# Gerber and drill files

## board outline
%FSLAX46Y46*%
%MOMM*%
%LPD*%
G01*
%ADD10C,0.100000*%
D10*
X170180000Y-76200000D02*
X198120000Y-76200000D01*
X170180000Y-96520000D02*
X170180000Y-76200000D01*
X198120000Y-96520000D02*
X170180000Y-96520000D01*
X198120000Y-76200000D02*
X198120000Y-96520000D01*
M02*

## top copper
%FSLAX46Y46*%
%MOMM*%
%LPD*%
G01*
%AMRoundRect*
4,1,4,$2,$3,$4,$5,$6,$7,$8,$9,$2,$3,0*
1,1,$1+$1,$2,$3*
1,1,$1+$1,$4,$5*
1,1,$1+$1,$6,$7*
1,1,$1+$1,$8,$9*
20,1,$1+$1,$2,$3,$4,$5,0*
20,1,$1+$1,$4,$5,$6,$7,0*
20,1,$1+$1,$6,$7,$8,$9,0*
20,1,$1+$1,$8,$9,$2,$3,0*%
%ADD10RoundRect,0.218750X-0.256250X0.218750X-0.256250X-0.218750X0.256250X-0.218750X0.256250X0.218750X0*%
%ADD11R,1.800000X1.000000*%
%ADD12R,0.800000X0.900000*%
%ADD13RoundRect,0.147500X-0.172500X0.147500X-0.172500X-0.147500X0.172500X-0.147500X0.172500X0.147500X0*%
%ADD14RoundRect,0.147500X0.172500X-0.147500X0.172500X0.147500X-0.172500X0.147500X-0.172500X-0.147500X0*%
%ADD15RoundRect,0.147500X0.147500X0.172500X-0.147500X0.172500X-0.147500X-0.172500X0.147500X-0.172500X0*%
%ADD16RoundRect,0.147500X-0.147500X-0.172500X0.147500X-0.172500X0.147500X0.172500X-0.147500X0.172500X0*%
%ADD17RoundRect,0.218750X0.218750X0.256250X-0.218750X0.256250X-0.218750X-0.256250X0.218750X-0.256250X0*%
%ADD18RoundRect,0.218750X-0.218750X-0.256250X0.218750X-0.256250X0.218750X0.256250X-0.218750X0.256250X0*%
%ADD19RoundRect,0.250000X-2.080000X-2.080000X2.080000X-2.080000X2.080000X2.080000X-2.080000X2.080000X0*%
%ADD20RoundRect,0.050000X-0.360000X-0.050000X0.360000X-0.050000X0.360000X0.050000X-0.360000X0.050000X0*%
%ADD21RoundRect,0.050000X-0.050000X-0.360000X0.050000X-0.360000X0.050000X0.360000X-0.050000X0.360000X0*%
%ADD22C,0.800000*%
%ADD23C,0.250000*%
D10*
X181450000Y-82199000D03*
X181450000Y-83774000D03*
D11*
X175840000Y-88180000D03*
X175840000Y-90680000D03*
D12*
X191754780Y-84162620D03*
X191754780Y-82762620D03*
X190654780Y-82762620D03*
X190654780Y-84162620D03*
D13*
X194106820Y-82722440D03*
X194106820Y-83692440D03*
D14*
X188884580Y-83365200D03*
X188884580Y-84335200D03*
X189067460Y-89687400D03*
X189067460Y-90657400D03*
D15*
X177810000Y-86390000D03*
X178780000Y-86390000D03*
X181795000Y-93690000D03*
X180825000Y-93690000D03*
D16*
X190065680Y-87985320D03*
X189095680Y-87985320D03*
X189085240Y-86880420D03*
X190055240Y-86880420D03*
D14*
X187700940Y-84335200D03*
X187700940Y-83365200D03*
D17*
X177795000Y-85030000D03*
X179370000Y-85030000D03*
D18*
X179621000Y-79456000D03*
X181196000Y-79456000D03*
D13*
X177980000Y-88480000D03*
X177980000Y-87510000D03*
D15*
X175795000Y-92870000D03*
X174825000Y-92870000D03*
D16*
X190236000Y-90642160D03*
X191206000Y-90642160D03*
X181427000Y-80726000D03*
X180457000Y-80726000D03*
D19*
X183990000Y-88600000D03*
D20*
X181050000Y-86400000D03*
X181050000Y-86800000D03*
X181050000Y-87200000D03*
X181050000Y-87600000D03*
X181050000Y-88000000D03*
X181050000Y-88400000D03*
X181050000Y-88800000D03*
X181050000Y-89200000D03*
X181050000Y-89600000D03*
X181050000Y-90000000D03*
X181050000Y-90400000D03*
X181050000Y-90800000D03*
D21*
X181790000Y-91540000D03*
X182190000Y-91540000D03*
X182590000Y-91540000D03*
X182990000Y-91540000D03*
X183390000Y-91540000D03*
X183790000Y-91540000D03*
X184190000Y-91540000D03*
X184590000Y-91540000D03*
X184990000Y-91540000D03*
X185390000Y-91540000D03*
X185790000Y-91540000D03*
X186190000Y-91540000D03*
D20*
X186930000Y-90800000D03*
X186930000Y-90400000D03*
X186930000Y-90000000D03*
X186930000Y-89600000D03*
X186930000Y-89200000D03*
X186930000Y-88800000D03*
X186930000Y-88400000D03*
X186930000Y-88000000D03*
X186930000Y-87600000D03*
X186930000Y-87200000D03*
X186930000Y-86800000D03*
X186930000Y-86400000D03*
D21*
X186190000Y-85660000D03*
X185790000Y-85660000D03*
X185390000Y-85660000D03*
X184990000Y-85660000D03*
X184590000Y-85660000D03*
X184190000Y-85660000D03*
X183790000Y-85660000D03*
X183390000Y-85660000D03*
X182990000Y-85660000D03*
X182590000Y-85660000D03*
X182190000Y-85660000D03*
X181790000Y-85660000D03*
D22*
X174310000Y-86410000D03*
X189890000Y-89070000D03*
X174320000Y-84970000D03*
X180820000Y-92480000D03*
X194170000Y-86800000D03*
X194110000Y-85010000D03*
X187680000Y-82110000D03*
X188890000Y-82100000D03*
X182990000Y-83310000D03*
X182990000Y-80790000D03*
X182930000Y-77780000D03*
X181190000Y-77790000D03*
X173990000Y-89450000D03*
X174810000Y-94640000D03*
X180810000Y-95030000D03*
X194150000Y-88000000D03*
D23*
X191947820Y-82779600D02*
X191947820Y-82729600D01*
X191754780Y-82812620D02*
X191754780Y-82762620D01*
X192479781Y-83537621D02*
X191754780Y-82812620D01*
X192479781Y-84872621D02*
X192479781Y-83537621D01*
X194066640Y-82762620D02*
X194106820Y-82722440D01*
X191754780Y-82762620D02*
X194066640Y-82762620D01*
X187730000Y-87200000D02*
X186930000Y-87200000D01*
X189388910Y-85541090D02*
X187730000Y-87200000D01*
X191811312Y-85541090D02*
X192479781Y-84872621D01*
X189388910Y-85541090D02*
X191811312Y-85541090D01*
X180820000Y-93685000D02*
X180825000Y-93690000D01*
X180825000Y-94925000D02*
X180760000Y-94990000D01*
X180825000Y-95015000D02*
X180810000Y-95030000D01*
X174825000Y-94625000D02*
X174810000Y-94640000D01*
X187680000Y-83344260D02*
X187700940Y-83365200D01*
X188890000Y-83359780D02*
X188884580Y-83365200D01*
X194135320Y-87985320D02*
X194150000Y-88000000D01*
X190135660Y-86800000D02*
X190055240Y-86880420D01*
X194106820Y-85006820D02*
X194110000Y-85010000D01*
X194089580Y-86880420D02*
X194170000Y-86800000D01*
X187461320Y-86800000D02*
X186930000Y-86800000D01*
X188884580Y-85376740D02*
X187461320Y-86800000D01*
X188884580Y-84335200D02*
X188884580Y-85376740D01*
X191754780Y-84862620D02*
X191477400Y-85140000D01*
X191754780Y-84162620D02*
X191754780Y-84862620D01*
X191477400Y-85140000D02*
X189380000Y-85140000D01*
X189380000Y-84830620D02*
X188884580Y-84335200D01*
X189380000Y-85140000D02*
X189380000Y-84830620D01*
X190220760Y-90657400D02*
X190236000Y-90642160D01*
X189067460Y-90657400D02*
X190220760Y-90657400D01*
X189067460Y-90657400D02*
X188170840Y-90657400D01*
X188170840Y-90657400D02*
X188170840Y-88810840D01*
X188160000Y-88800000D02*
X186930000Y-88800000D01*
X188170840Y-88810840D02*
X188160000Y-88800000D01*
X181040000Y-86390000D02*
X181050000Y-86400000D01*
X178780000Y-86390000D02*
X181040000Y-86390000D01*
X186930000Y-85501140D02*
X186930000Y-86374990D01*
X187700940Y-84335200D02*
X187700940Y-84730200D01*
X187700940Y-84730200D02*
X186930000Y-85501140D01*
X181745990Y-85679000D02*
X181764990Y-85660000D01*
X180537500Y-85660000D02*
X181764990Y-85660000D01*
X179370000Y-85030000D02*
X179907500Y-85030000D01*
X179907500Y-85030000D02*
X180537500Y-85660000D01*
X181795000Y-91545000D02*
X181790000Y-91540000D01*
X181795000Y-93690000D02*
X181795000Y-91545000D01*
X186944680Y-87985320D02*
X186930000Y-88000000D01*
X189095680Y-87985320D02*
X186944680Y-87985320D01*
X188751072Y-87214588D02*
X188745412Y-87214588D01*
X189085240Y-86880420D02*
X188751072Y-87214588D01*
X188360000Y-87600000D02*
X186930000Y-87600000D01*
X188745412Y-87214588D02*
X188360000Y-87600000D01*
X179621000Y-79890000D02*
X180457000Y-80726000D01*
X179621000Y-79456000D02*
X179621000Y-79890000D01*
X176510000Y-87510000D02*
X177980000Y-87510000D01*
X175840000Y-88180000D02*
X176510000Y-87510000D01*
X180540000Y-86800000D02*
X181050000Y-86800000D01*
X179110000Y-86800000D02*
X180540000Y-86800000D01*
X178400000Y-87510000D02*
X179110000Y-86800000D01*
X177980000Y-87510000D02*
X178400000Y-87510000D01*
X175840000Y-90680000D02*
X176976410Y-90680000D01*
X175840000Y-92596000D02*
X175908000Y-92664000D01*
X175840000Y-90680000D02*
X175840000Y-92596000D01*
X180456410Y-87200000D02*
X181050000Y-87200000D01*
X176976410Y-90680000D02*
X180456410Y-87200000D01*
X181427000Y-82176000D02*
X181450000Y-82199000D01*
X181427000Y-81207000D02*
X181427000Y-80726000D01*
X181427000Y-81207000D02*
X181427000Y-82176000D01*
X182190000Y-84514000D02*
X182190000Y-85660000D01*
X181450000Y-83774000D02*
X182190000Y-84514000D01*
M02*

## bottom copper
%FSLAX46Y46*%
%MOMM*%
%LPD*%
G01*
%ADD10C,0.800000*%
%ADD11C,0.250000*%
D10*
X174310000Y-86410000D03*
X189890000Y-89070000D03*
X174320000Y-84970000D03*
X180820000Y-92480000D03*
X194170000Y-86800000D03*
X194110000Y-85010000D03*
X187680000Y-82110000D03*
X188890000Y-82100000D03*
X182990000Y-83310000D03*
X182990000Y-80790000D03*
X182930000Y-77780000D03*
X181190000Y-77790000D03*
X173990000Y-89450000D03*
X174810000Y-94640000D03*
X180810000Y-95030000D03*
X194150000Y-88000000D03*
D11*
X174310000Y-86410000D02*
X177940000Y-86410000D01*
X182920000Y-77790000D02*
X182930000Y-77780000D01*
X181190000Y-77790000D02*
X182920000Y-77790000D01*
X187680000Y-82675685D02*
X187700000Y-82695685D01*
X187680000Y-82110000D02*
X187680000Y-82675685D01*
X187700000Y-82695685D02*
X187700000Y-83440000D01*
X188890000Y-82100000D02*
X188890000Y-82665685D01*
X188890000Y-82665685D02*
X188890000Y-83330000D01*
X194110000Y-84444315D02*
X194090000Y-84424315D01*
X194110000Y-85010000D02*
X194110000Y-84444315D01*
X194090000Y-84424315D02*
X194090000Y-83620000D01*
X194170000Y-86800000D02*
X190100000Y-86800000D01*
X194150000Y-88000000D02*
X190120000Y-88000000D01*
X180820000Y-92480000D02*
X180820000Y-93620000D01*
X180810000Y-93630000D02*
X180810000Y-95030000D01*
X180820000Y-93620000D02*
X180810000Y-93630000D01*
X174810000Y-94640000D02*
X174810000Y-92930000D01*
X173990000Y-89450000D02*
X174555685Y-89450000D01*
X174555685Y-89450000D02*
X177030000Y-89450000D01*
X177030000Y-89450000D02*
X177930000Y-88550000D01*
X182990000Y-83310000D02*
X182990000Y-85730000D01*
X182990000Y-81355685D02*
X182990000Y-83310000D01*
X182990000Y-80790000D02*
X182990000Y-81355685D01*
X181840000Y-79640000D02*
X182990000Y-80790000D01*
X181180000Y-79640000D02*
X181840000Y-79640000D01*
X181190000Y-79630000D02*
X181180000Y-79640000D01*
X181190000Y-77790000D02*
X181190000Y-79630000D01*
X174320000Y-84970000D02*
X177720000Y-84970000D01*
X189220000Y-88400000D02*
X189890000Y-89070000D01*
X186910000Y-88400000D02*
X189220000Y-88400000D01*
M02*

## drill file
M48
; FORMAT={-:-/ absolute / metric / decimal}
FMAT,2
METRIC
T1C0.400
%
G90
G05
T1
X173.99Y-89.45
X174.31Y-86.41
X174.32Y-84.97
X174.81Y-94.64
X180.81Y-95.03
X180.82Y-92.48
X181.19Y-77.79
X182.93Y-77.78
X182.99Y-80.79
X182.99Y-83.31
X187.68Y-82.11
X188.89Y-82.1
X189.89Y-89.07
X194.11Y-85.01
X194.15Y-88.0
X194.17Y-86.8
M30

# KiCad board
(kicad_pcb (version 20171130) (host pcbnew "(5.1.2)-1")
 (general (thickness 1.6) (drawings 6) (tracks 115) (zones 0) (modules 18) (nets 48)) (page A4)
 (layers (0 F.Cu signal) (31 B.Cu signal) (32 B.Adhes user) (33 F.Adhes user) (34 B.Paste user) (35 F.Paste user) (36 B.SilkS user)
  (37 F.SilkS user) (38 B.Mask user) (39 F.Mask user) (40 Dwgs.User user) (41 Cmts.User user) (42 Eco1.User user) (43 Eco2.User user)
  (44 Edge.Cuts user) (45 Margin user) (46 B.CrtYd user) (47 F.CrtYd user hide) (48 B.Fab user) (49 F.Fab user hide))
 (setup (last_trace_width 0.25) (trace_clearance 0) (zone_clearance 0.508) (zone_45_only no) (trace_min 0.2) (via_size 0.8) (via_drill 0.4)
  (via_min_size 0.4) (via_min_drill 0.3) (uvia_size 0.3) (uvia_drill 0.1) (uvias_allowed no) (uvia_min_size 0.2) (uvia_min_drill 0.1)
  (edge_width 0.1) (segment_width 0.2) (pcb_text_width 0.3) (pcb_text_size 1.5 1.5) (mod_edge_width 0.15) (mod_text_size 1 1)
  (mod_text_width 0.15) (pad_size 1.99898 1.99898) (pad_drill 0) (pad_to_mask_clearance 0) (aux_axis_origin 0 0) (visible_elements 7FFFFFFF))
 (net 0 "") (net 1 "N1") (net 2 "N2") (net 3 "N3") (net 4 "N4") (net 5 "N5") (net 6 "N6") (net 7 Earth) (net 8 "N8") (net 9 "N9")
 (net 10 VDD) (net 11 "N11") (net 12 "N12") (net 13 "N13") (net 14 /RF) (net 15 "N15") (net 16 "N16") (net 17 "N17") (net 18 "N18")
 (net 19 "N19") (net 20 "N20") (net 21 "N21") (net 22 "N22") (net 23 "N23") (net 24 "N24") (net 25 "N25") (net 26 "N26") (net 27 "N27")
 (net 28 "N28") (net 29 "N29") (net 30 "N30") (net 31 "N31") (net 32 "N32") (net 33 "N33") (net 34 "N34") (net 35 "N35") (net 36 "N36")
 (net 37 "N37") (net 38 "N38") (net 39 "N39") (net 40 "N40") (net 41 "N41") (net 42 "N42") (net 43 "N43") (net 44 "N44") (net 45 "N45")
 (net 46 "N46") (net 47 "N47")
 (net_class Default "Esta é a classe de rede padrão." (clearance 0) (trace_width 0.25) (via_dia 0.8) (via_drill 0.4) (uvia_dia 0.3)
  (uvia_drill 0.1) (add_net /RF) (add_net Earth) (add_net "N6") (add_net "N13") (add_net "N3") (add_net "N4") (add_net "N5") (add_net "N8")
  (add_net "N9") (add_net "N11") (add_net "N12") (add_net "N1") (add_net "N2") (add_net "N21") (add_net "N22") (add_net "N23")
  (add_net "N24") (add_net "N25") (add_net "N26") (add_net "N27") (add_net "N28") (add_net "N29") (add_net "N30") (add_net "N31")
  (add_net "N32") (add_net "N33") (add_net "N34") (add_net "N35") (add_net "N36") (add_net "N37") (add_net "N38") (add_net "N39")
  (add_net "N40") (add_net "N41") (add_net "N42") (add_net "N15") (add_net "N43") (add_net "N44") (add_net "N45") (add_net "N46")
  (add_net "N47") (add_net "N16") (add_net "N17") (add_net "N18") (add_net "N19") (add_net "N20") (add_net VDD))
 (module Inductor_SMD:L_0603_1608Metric (layer F.Cu) (at 181.45 82.9865 270)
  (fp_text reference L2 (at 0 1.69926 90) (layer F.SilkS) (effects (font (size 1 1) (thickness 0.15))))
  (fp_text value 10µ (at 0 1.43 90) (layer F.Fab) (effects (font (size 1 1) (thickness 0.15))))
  (pad 1 smd roundrect (at -0.7875 0 270) (size 0.875 0.95) (layers F.Cu F.Paste F.Mask) (roundrect_rratio 0.25) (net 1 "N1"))
  (pad 2 smd roundrect (at 0.7875 0 270) (size 0.875 0.95) (layers F.Cu F.Paste F.Mask) (roundrect_rratio 0.25) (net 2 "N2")))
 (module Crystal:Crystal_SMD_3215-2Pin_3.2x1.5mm (layer F.Cu) (at 175.84 89.43 90)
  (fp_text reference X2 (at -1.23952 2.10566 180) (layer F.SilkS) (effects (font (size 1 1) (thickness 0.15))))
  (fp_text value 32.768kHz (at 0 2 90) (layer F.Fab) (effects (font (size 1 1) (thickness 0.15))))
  (pad 1 smd rect (at 1.25 0 90) (size 1 1.8) (layers F.Cu F.Paste F.Mask) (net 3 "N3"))
  (pad 2 smd rect (at -1.25 0 90) (size 1 1.8) (layers F.Cu F.Paste F.Mask) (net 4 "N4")))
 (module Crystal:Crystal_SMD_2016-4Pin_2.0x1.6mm (layer F.Cu) (at 191.20478 83.46262 90)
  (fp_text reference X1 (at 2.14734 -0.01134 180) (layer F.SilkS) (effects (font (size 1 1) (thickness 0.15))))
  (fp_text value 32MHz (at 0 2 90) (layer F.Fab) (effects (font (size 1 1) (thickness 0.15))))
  (pad 1 smd rect (at -0.7 0.55 90) (size 0.9 0.8) (layers F.Cu F.Paste F.Mask) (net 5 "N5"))
  (pad 2 smd rect (at 0.7 0.55 90) (size 0.9 0.8) (layers F.Cu F.Paste F.Mask) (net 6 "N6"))
  (pad 3 smd rect (at 0.7 -0.55 90) (size 0.9 0.8) (layers F.Cu F.Paste F.Mask))
  (pad 4 smd rect (at -0.7 -0.55 90) (size 0.9 0.8) (layers F.Cu F.Paste F.Mask)))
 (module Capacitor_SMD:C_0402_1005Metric (layer F.Cu) (at 194.10682 83.20744 270)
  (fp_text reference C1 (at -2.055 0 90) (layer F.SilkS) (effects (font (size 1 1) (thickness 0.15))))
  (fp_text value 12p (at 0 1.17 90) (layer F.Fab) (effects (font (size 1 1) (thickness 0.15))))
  (pad 1 smd roundrect (at -0.485 0 270) (size 0.59 0.64) (layers F.Cu F.Paste F.Mask) (roundrect_rratio 0.25) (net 6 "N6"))
  (pad 2 smd roundrect (at 0.485 0 270) (size 0.59 0.64) (layers F.Cu F.Paste F.Mask) (roundrect_rratio 0.25) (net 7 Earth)))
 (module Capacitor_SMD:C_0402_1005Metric (layer F.Cu) (at 188.88458 83.8502 90)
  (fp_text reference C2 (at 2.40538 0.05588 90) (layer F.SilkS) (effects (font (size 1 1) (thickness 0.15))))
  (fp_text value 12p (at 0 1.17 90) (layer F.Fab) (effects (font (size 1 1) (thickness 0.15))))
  (pad 2 smd roundrect (at 0.485 0 90) (size 0.59 0.64) (layers F.Cu F.Paste F.Mask) (roundrect_rratio 0.25) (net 7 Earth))
  (pad 1 smd roundrect (at -0.485 0 90) (size 0.59 0.64) (layers F.Cu F.Paste F.Mask) (roundrect_rratio 0.25) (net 5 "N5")))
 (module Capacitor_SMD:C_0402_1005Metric (layer F.Cu) (at 189.06746 90.1724 90)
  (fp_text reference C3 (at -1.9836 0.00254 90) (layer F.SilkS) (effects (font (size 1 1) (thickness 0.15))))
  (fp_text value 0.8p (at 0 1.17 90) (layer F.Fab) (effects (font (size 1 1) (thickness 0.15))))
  (pad 2 smd roundrect (at 0.485 0 90) (size 0.59 0.64) (layers F.Cu F.Paste F.Mask) (roundrect_rratio 0.25) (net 7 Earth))
  (pad 1 smd roundrect (at -0.485 0 90) (size 0.59 0.64) (layers F.Cu F.Paste F.Mask) (roundrect_rratio 0.25) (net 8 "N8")))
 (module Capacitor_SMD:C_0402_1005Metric (layer F.Cu) (at 178.295 86.39 180)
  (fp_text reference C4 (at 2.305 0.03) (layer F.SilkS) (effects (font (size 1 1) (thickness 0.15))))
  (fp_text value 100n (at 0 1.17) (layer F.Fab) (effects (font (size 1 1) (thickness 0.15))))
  (pad 2 smd roundrect (at 0.485 0 180) (size 0.59 0.64) (layers F.Cu F.Paste F.Mask) (roundrect_rratio 0.25) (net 7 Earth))
  (pad 1 smd roundrect (at -0.485 0 180) (size 0.59 0.64) (layers F.Cu F.Paste F.Mask) (roundrect_rratio 0.25) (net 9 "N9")))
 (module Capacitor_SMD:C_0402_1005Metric (layer F.Cu) (at 181.31 93.69 180)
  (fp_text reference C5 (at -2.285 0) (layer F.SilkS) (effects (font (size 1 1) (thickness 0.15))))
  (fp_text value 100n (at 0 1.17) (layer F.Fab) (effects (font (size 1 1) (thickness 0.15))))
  (pad 1 smd roundrect (at -0.485 0 180) (size 0.59 0.64) (layers F.Cu F.Paste F.Mask) (roundrect_rratio 0.25) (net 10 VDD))
  (pad 2 smd roundrect (at 0.485 0 180) (size 0.59 0.64) (layers F.Cu F.Paste F.Mask) (roundrect_rratio 0.25) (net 7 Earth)))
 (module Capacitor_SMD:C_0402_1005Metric (layer F.Cu) (at 189.58068 87.98532)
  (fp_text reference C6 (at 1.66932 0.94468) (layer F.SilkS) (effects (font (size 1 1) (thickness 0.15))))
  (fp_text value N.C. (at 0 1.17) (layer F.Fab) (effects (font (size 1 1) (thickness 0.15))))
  (pad 2 smd roundrect (at 0.485 0) (size 0.59 0.64) (layers F.Cu F.Paste F.Mask) (roundrect_rratio 0.25) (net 7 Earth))
  (pad 1 smd roundrect (at -0.485 0) (size 0.59 0.64) (layers F.Cu F.Paste F.Mask) (roundrect_rratio 0.25) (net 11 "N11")))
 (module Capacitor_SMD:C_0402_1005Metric (layer F.Cu) (at 189.57024 86.88042)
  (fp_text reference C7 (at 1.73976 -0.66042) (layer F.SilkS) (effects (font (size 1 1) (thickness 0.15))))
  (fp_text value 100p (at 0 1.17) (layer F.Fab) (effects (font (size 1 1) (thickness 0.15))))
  (pad 1 smd roundrect (at -0.485 0) (size 0.59 0.64) (layers F.Cu F.Paste F.Mask) (roundrect_rratio 0.25) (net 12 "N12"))
  (pad 2 smd roundrect (at 0.485 0) (size 0.59 0.64) (layers F.Cu F.Paste F.Mask) (roundrect_rratio 0.25) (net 7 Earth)))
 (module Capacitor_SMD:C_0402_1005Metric (layer F.Cu) (at 187.70094 83.8502 90)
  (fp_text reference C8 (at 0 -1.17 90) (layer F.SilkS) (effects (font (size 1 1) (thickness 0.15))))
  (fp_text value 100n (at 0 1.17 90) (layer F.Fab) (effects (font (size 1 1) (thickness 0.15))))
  (pad 1 smd roundrect (at -0.485 0 90) (size 0.59 0.64) (layers F.Cu F.Paste F.Mask) (roundrect_rratio 0.25) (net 10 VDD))
  (pad 2 smd roundrect (at 0.485 0 90) (size 0.59 0.64) (layers F.Cu F.Paste F.Mask) (roundrect_rratio 0.25) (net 7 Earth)))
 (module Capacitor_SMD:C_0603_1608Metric (layer F.Cu) (at 178.5825 85.03 180)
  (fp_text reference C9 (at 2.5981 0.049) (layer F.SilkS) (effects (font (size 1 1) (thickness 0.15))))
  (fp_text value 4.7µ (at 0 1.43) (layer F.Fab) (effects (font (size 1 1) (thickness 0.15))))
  (pad 2 smd roundrect (at 0.7875 0 180) (size 0.875 0.95) (layers F.Cu F.Paste F.Mask) (roundrect_rratio 0.25) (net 7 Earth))
  (pad 1 smd roundrect (at -0.7875 0 180) (size 0.875 0.95) (layers F.Cu F.Paste F.Mask) (roundrect_rratio 0.25) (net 10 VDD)))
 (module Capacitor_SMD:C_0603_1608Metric (layer F.Cu) (at 180.4085 79.456)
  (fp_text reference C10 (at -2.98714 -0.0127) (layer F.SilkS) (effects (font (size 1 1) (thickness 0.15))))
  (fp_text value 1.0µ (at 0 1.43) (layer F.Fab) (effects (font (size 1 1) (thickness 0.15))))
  (pad 1 smd roundrect (at -0.7875 0) (size 0.875 0.95) (layers F.Cu F.Paste F.Mask) (roundrect_rratio 0.25) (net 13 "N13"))
  (pad 2 smd roundrect (at 0.7875 0) (size 0.875 0.95) (layers F.Cu F.Paste F.Mask) (roundrect_rratio 0.25) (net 7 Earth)))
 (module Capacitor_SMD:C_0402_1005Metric (layer F.Cu) (at 177.98 87.995 270)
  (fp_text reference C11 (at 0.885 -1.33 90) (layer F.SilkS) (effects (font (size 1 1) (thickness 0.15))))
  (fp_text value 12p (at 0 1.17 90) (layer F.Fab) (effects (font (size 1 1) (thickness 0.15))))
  (pad 2 smd roundrect (at 0.485 0 270) (size 0.59 0.64) (layers F.Cu F.Paste F.Mask) (roundrect_rratio 0.25) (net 7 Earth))
  (pad 1 smd roundrect (at -0.485 0 270) (size 0.59 0.64) (layers F.Cu F.Paste F.Mask) (roundrect_rratio 0.25) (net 3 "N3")))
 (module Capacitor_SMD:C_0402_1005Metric (layer F.Cu) (at 175.31 92.87 180)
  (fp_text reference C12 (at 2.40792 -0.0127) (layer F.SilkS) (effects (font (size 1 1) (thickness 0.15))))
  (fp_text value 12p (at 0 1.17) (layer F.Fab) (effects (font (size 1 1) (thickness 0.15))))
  (pad 1 smd roundrect (at -0.485 0 180) (size 0.59 0.64) (layers F.Cu F.Paste F.Mask) (roundrect_rratio 0.25) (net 4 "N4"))
  (pad 2 smd roundrect (at 0.485 0 180) (size 0.59 0.64) (layers F.Cu F.Paste F.Mask) (roundrect_rratio 0.25) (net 7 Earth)))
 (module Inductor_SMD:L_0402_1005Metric (layer F.Cu) (at 190.721 90.64216)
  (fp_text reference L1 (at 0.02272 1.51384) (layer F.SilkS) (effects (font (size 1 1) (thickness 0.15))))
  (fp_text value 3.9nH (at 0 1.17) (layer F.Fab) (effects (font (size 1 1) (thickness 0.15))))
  (pad 1 smd roundrect (at -0.485 0) (size 0.59 0.64) (layers F.Cu F.Paste F.Mask) (roundrect_rratio 0.25) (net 8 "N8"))
  (pad 2 smd roundrect (at 0.485 0) (size 0.59 0.64) (layers F.Cu F.Paste F.Mask) (roundrect_rratio 0.25) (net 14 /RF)))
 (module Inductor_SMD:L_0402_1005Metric (layer F.Cu) (at 180.942 80.726)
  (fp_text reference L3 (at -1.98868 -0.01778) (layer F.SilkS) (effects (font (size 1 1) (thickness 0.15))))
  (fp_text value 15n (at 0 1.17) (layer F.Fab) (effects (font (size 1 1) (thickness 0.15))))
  (pad 2 smd roundrect (at 0.485 0) (size 0.59 0.64) (layers F.Cu F.Paste F.Mask) (roundrect_rratio 0.25) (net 1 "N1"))
  (pad 1 smd roundrect (at -0.485 0) (size 0.59 0.64) (layers F.Cu F.Paste F.Mask) (roundrect_rratio 0.25) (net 13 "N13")))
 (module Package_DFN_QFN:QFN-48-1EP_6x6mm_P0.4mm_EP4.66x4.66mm (layer F.Cu) (at 183.99 88.6)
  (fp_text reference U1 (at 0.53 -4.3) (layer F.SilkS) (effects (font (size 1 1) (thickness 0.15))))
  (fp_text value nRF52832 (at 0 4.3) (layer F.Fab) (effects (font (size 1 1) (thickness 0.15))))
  (pad 49 smd roundrect (at 0 0) (size 4.66 4.66) (layers F.Cu F.Mask) (roundrect_rratio 0.053648))
  (pad "" smd roundrect (at -1.55 -1.55) (size 1.25 1.25) (layers F.Paste) (roundrect_rratio 0.2))
  (pad "" smd roundrect (at -1.55 0) (size 1.25 1.25) (layers F.Paste) (roundrect_rratio 0.2))
  (pad "" smd roundrect (at -1.55 1.55) (size 1.25 1.25) (layers F.Paste) (roundrect_rratio 0.2))
  (pad "" smd roundrect (at 0 -1.55) (size 1.25 1.25) (layers F.Paste) (roundrect_rratio 0.2))
  (pad "" smd roundrect (at 0 0) (size 1.25 1.25) (layers F.Paste) (roundrect_rratio 0.2))
  (pad "" smd roundrect (at 0 1.55) (size 1.25 1.25) (layers F.Paste) (roundrect_rratio 0.2))
  (pad "" smd roundrect (at 1.55 -1.55) (size 1.25 1.25) (layers F.Paste) (roundrect_rratio 0.2))
  (pad "" smd roundrect (at 1.55 0) (size 1.25 1.25) (layers F.Paste) (roundrect_rratio 0.2))
  (pad "" smd roundrect (at 1.55 1.55) (size 1.25 1.25) (layers F.Paste) (roundrect_rratio 0.2))
  (pad 1 smd roundrect (at -2.94 -2.2) (size 0.82 0.2) (layers F.Cu F.Paste F.Mask) (roundrect_rratio 0.25) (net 9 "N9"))
  (pad 2 smd roundrect (at -2.94 -1.8) (size 0.82 0.2) (layers F.Cu F.Paste F.Mask) (roundrect_rratio 0.25) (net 3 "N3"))
  (pad 3 smd roundrect (at -2.94 -1.4) (size 0.82 0.2) (layers F.Cu F.Paste F.Mask) (roundrect_rratio 0.25) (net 4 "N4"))
  (pad 4 smd roundrect (at -2.94 -1) (size 0.82 0.2) (layers F.Cu F.Paste F.Mask) (roundrect_rratio 0.25) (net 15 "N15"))
  (pad 5 smd roundrect (at -2.94 -0.6) (size 0.82 0.2) (layers F.Cu F.Paste F.Mask) (roundrect_rratio 0.25) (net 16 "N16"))
  (pad 6 smd roundrect (at -2.94 -0.2) (size 0.82 0.2) (layers F.Cu F.Paste F.Mask) (roundrect_rratio 0.25) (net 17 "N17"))
  (pad 7 smd roundrect (at -2.94 0.2) (size 0.82 0.2) (layers F.Cu F.Paste F.Mask) (roundrect_rratio 0.25) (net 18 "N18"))
  (pad 8 smd roundrect (at -2.94 0.6) (size 0.82 0.2) (layers F.Cu F.Paste F.Mask) (roundrect_rratio 0.25) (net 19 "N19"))
  (pad 9 smd roundrect (at -2.94 1) (size 0.82 0.2) (layers F.Cu F.Paste F.Mask) (roundrect_rratio 0.25) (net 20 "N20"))
  (pad 10 smd roundrect (at -2.94 1.4) (size 0.82 0.2) (layers F.Cu F.Paste F.Mask) (roundrect_rratio 0.25) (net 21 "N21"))
  (pad 11 smd roundrect (at -2.94 1.8) (size 0.82 0.2) (layers F.Cu F.Paste F.Mask) (roundrect_rratio 0.25) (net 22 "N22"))
  (pad 12 smd roundrect (at -2.94 2.2) (size 0.82 0.2) (layers F.Cu F.Paste F.Mask) (roundrect_rratio 0.25) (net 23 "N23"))
  (pad 13 smd roundrect (at -2.2 2.94) (size 0.2 0.82) (layers F.Cu F.Paste F.Mask) (roundrect_rratio 0.25) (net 10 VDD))
  (pad 14 smd roundrect (at -1.8 2.94) (size 0.2 0.82) (layers F.Cu F.Paste F.Mask) (roundrect_rratio 0.25) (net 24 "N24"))
  (pad 15 smd roundrect (at -1.4 2.94) (size 0.2 0.82) (layers F.Cu F.Paste F.Mask) (roundrect_rratio 0.25) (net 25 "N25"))
  (pad 16 smd roundrect (at -1 2.94) (size 0.2 0.82) (layers F.Cu F.Paste F.Mask) (roundrect_rratio 0.25) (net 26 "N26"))
  (pad 17 smd roundrect (at -0.6 2.94) (size 0.2 0.82) (layers F.Cu F.Paste F.Mask) (roundrect_rratio 0.25) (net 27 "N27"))
  (pad 18 smd roundrect (at -0.2 2.94) (size 0.2 0.82) (layers F.Cu F.Paste F.Mask) (roundrect_rratio 0.25) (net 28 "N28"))
  (pad 19 smd roundrect (at 0.2 2.94) (size 0.2 0.82) (layers F.Cu F.Paste F.Mask) (roundrect_rratio 0.25) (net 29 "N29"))
  (pad 20 smd roundrect (at 0.6 2.94) (size 0.2 0.82) (layers F.Cu F.Paste F.Mask) (roundrect_rratio 0.25) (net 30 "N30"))
  (pad 21 smd roundrect (at 1 2.94) (size 0.2 0.82) (layers F.Cu F.Paste F.Mask) (roundrect_rratio 0.25) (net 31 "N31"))
  (pad 22 smd roundrect (at 1.4 2.94) (size 0.2 0.82) (layers F.Cu F.Paste F.Mask) (roundrect_rratio 0.25) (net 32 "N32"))
  (pad 23 smd roundrect (at 1.8 2.94) (size 0.2 0.82) (layers F.Cu F.Paste F.Mask) (roundrect_rratio 0.25) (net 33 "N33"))
  (pad 24 smd roundrect (at 2.2 2.94) (size 0.2 0.82) (layers F.Cu F.Paste F.Mask) (roundrect_rratio 0.25) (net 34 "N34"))
  (pad 25 smd roundrect (at 2.94 2.2) (size 0.82 0.2) (layers F.Cu F.Paste F.Mask) (roundrect_rratio 0.25) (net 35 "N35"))
  (pad 26 smd roundrect (at 2.94 1.8) (size 0.82 0.2) (layers F.Cu F.Paste F.Mask) (roundrect_rratio 0.25) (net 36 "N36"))
  (pad 27 smd roundrect (at 2.94 1.4) (size 0.82 0.2) (layers F.Cu F.Paste F.Mask) (roundrect_rratio 0.25) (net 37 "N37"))
  (pad 28 smd roundrect (at 2.94 1) (size 0.82 0.2) (layers F.Cu F.Paste F.Mask) (roundrect_rratio 0.25) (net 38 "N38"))
  (pad 29 smd roundrect (at 2.94 0.6) (size 0.82 0.2) (layers F.Cu F.Paste F.Mask) (roundrect_rratio 0.25) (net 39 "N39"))
  (pad 30 smd roundrect (at 2.94 0.2) (size 0.82 0.2) (layers F.Cu F.Paste F.Mask) (roundrect_rratio 0.25) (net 8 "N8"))
  (pad 31 smd roundrect (at 2.94 -0.2) (size 0.82 0.2) (layers F.Cu F.Paste F.Mask) (roundrect_rratio 0.25) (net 7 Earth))
  (pad 32 smd roundrect (at 2.94 -0.6) (size 0.82 0.2) (layers F.Cu F.Paste F.Mask) (roundrect_rratio 0.25) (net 11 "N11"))
  (pad 33 smd roundrect (at 2.94 -1) (size 0.82 0.2) (layers F.Cu F.Paste F.Mask) (roundrect_rratio 0.25) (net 12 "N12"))
  (pad 34 smd roundrect (at 2.94 -1.4) (size 0.82 0.2) (layers F.Cu F.Paste F.Mask) (roundrect_rratio 0.25) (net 6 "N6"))
  (pad 35 smd roundrect (at 2.94 -1.8) (size 0.82 0.2) (layers F.Cu F.Paste F.Mask) (roundrect_rratio 0.25) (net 5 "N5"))
  (pad 36 smd roundrect (at 2.94 -2.2) (size 0.82 0.2) (layers F.Cu F.Paste F.Mask) (roundrect_rratio 0.25) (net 10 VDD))
  (pad 37 smd roundrect (at 2.2 -2.94) (size 0.2 0.82) (layers F.Cu F.Paste F.Mask) (roundrect_rratio 0.25) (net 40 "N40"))
  (pad 38 smd roundrect (at 1.8 -2.94) (size 0.2 0.82) (layers F.Cu F.Paste F.Mask) (roundrect_rratio 0.25) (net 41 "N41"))
  (pad 39 smd roundrect (at 1.4 -2.94) (size 0.2 0.82) (layers F.Cu F.Paste F.Mask) (roundrect_rratio 0.25) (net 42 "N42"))
  (pad 40 smd roundrect (at 1 -2.94) (size 0.2 0.82) (layers F.Cu F.Paste F.Mask) (roundrect_rratio 0.25) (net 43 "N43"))
  (pad 41 smd roundrect (at 0.6 -2.94) (size 0.2 0.82) (layers F.Cu F.Paste F.Mask) (roundrect_rratio 0.25) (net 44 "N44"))
  (pad 42 smd roundrect (at 0.2 -2.94) (size 0.2 0.82) (layers F.Cu F.Paste F.Mask) (roundrect_rratio 0.25) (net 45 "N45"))
  (pad 43 smd roundrect (at -0.2 -2.94) (size 0.2 0.82) (layers F.Cu F.Paste F.Mask) (roundrect_rratio 0.25) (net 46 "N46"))
  (pad 44 smd roundrect (at -0.6 -2.94) (size 0.2 0.82) (layers F.Cu F.Paste F.Mask) (roundrect_rratio 0.25) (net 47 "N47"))
  (pad 45 smd roundrect (at -1 -2.94) (size 0.2 0.82) (layers F.Cu F.Paste F.Mask) (roundrect_rratio 0.25) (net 7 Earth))
  (pad 46 smd roundrect (at -1.4 -2.94) (size 0.2 0.82) (layers F.Cu F.Paste F.Mask) (roundrect_rratio 0.25) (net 13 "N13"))
  (pad 47 smd roundrect (at -1.8 -2.94) (size 0.2 0.82) (layers F.Cu F.Paste F.Mask) (roundrect_rratio 0.25) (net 2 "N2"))
  (pad 48 smd roundrect (at -2.2 -2.94) (size 0.2 0.82) (layers F.Cu F.Paste F.Mask) (roundrect_rratio 0.25) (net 10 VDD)))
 (gr_line (start 170.18 76.2) (end 198.12 76.2) (layer Edge.Cuts) (width 0.1))
 (gr_line (start 170.18 96.52) (end 170.18 76.2) (layer Edge.Cuts) (width 0.1))
 (gr_line (start 198.12 96.52) (end 170.18 96.52) (layer Edge.Cuts) (width 0.1))
 (gr_line (start 198.12 76.2) (end 198.12 96.52) (layer Edge.Cuts) (width 0.1))
 (via (at 174.31 86.41) (size 0.8) (drill 0.4) (layers F.Cu B.Cu) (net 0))
 (segment (start 174.31 86.41) (end 177.94 86.41) (width 0.25) (layer B.Cu) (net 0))
 (via (at 189.89 89.07) (size 0.8) (drill 0.4) (layers F.Cu B.Cu) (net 7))
 (via (at 174.32 84.97) (size 0.8) (drill 0.4) (layers F.Cu B.Cu) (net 7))
 (segment (start 191.94782 82.7796) (end 191.94782 82.7296) (width 0.25) (layer F.Cu) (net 6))
 (segment (start 191.75478 82.81262) (end 191.75478 82.76262) (width 0.25) (layer F.Cu) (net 6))
 (segment (start 192.479781 83.537621) (end 191.75478 82.81262) (width 0.25) (layer F.Cu) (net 6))
 (segment (start 192.479781 84.872621) (end 192.479781 83.537621) (width 0.25) (layer F.Cu) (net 6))
 (segment (start 194.06664 82.76262) (end 194.10682 82.72244) (width 0.25) (layer F.Cu) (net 6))
 (segment (start 191.75478 82.76262) (end 194.06664 82.76262) (width 0.25) (layer F.Cu) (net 6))
 (segment (start 187.73 87.2) (end 186.93 87.2) (width 0.25) (layer F.Cu) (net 6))
 (segment (start 189.38891 85.54109) (end 187.73 87.2) (width 0.25) (layer F.Cu) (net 6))
 (segment (start 191.811312 85.54109) (end 192.479781 84.872621) (width 0.25) (layer F.Cu) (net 6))
 (segment (start 189.38891 85.54109) (end 191.811312 85.54109) (width 0.25) (layer F.Cu) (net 6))
 (via (at 180.82 92.48) (size 0.8) (drill 0.4) (layers F.Cu B.Cu) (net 7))
 (via (at 194.17 86.8) (size 0.8) (drill 0.4) (layers F.Cu B.Cu) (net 7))
 (via (at 194.11 85.01) (size 0.8) (drill 0.4) (layers F.Cu B.Cu) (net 7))
 (via (at 187.68 82.11) (size 0.8) (drill 0.4) (layers F.Cu B.Cu) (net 7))
 (via (at 188.89 82.1) (size 0.8) (drill 0.4) (layers F.Cu B.Cu) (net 7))
 (via (at 182.99 83.31) (size 0.8) (drill 0.4) (layers F.Cu B.Cu) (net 7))
 (via (at 182.99 80.79) (size 0.8) (drill 0.4) (layers F.Cu B.Cu) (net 7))
 (via (at 182.93 77.78) (size 0.8) (drill 0.4) (layers F.Cu B.Cu) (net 7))
 (via (at 181.19 77.79) (size 0.8) (drill 0.4) (layers F.Cu B.Cu) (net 7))
 (via (at 173.99 89.45) (size 0.8) (drill 0.4) (layers F.Cu B.Cu) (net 7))
 (via (at 174.81 94.64) (size 0.8) (drill 0.4) (layers F.Cu B.Cu) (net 7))
 (via (at 180.81 95.03) (size 0.8) (drill 0.4) (layers F.Cu B.Cu) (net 7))
 (segment (start 180.82 93.685) (end 180.825 93.69) (width 0.25) (layer F.Cu) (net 7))
 (segment (start 180.825 94.925) (end 180.76 94.99) (width 0.25) (layer F.Cu) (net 7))
 (segment (start 180.825 95.015) (end 180.81 95.03) (width 0.25) (layer F.Cu) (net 7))
 (segment (start 174.825 94.625) (end 174.81 94.64) (width 0.25) (layer F.Cu) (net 7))
 (segment (start 187.68 83.34426) (end 187.70094 83.3652) (width 0.25) (layer F.Cu) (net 7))
 (segment (start 188.89 83.35978) (end 188.88458 83.3652) (width 0.25) (layer F.Cu) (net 7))
 (via (at 194.15 88) (size 0.8) (drill 0.4) (layers F.Cu B.Cu) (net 7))
 (segment (start 194.13532 87.98532) (end 194.15 88) (width 0.25) (layer F.Cu) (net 7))
 (segment (start 190.13566 86.8) (end 190.05524 86.88042) (width 0.25) (layer F.Cu) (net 7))
 (segment (start 182.92 77.79) (end 182.93 77.78) (width 0.25) (layer B.Cu) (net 7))
 (segment (start 181.19 77.79) (end 182.92 77.79) (width 0.25) (layer B.Cu) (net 7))
 (segment (start 187.68 82.675685) (end 187.7 82.695685) (width 0.25) (layer B.Cu) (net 7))
 (segment (start 187.68 82.11) (end 187.68 82.675685) (width 0.25) (layer B.Cu) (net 7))
 (segment (start 187.7 82.695685) (end 187.7 83.44) (width 0.25) (layer B.Cu) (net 7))
 (segment (start 188.89 82.1) (end 188.89 82.665685) (width 0.25) (layer B.Cu) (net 7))
 (segment (start 188.89 82.665685) (end 188.89 83.33) (width 0.25) (layer B.Cu) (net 7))
 (segment (start 194.10682 85.00682) (end 194.11 85.01) (width 0.25) (layer F.Cu) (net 7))
 (segment (start 194.08958 86.88042) (end 194.17 86.8) (width 0.25) (layer F.Cu) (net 7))
 (segment (start 194.11 84.444315) (end 194.09 84.424315) (width 0.25) (layer B.Cu) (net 7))
 (segment (start 194.11 85.01) (end 194.11 84.444315) (width 0.25) (layer B.Cu) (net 7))
 (segment (start 194.09 84.424315) (end 194.09 83.62) (width 0.25) (layer B.Cu) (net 7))
 (segment (start 194.17 86.8) (end 190.1 86.8) (width 0.25) (layer B.Cu) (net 7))
 (segment (start 194.15 88) (end 190.12 88) (width 0.25) (layer B.Cu) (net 7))
 (segment (start 180.82 92.48) (end 180.82 93.62) (width 0.25) (layer B.Cu) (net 7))
 (segment (start 180.81 93.63) (end 180.81 95.03) (width 0.25) (layer B.Cu) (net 7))
 (segment (start 180.82 93.62) (end 180.81 93.63) (width 0.25) (layer B.Cu) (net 7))
 (segment (start 174.81 94.64) (end 174.81 92.93) (width 0.25) (layer B.Cu) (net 7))
 (segment (start 173.99 89.45) (end 174.555685 89.45) (width 0.25) (layer B.Cu) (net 7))
 (segment (start 174.555685 89.45) (end 177.03 89.45) (width 0.25) (layer B.Cu) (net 7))
 (segment (start 177.03 89.45) (end 177.93 88.55) (width 0.25) (layer B.Cu) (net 7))
 (segment (start 182.99 83.31) (end 182.99 85.73) (width 0.25) (layer B.Cu) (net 7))
 (segment (start 182.99 81.355685) (end 182.99 83.31) (width 0.25) (layer B.Cu) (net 7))
 (segment (start 182.99 80.79) (end 182.99 81.355685) (width 0.25) (layer B.Cu) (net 7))
 (segment (start 181.84 79.64) (end 182.99 80.79) (width 0.25) (layer B.Cu) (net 7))
 (segment (start 181.18 79.64) (end 181.84 79.64) (width 0.25) (layer B.Cu) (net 7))
 (segment (start 181.19 79.63) (end 181.18 79.64) (width 0.25) (layer B.Cu) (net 7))
 (segment (start 181.19 77.79) (end 181.19 79.63) (width 0.25) (layer B.Cu) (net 7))
 (segment (start 174.32 84.97) (end 177.72 84.97) (width 0.25) (layer B.Cu) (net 7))
 (segment (start 189.22 88.4) (end 189.89 89.07) (width 0.25) (layer B.Cu) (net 7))
 (segment (start 186.91 88.4) (end 189.22 88.4) (width 0.25) (layer B.Cu) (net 7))
 (segment (start 187.46132 86.8) (end 186.93 86.8) (width 0.25) (layer F.Cu) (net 5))
 (segment (start 188.88458 85.37674) (end 187.46132 86.8) (width 0.25) (layer F.Cu) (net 5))
 (segment (start 188.88458 84.3352) (end 188.88458 85.37674) (width 0.25) (layer F.Cu) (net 5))
 (segment (start 191.75478 84.86262) (end 191.4774 85.14) (width 0.25) (layer F.Cu) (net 5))
 (segment (start 191.75478 84.16262) (end 191.75478 84.86262) (width 0.25) (layer F.Cu) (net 5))
 (segment (start 191.4774 85.14) (end 189.38 85.14) (width 0.25) (layer F.Cu) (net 5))
 (segment (start 189.38 84.83062) (end 188.88458 84.3352) (width 0.25) (layer F.Cu) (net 5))
 (segment (start 189.38 85.14) (end 189.38 84.83062) (width 0.25) (layer F.Cu) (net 5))
 (segment (start 190.22076 90.6574) (end 190.236 90.64216) (width 0.25) (layer F.Cu) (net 8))
 (segment (start 189.06746 90.6574) (end 190.22076 90.6574) (width 0.25) (layer F.Cu) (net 8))
 (segment (start 189.06746 90.6574) (end 188.17084 90.6574) (width 0.25) (layer F.Cu) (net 8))
 (segment (start 188.17084 90.6574) (end 188.17084 88.81084) (width 0.25) (layer F.Cu) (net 8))
 (segment (start 188.16 88.8) (end 186.93 88.8) (width 0.25) (layer F.Cu) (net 8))
 (segment (start 188.17084 88.81084) (end 188.16 88.8) (width 0.25) (layer F.Cu) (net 8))
 (segment (start 181.04 86.39) (end 181.05 86.4) (width 0.25) (layer F.Cu) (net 9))
 (segment (start 178.78 86.39) (end 181.04 86.39) (width 0.25) (layer F.Cu) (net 9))
 (segment (start 186.93 85.50114) (end 186.93 86.37499) (width 0.25) (layer F.Cu) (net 10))
 (segment (start 187.70094 84.3352) (end 187.70094 84.7302) (width 0.25) (layer F.Cu) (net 10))
 (segment (start 187.70094 84.7302) (end 186.93 85.50114) (width 0.25) (layer F.Cu) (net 10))
 (segment (start 181.74599 85.679) (end 181.76499 85.66) (width 0.25) (layer F.Cu) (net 10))
 (segment (start 180.5375 85.66) (end 181.76499 85.66) (width 0.25) (layer F.Cu) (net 10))
 (segment (start 179.37 85.03) (end 179.9075 85.03) (width 0.25) (layer F.Cu) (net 10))
 (segment (start 179.9075 85.03) (end 180.5375 85.66) (width 0.25) (layer F.Cu) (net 10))
 (segment (start 181.795 91.545) (end 181.79 91.54) (width 0.25) (layer F.Cu) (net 10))
 (segment (start 181.795 93.69) (end 181.795 91.545) (width 0.25) (layer F.Cu) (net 10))
 (segment (start 186.94468 87.98532) (end 186.93 88) (width 0.25) (layer F.Cu) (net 11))
 (segment (start 189.09568 87.98532) (end 186.94468 87.98532) (width 0.25) (layer F.Cu) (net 11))
 (segment (start 188.751072 87.214588) (end 188.745412 87.214588) (width 0.25) (layer F.Cu) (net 12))
 (segment (start 189.08524 86.88042) (end 188.751072 87.214588) (width 0.25) (layer F.Cu) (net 12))
 (segment (start 188.36 87.6) (end 186.93 87.6) (width 0.25) (layer F.Cu) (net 12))
 (segment (start 188.745412 87.214588) (end 188.36 87.6) (width 0.25) (layer F.Cu) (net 12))
 (segment (start 179.621 79.89) (end 180.457 80.726) (width 0.25) (layer F.Cu) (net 13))
 (segment (start 179.621 79.456) (end 179.621 79.89) (width 0.25) (layer F.Cu) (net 13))
 (segment (start 176.51 87.51) (end 177.98 87.51) (width 0.25) (layer F.Cu) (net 3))
 (segment (start 175.84 88.18) (end 176.51 87.51) (width 0.25) (layer F.Cu) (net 3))
 (segment (start 180.54 86.8) (end 181.05 86.8) (width 0.25) (layer F.Cu) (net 3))
 (segment (start 179.11 86.8) (end 180.54 86.8) (width 0.25) (layer F.Cu) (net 3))
 (segment (start 178.4 87.51) (end 179.11 86.8) (width 0.25) (layer F.Cu) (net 3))
 (segment (start 177.98 87.51) (end 178.4 87.51) (width 0.25) (layer F.Cu) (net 3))
 (segment (start 175.84 90.68) (end 176.97641 90.68) (width 0.25) (layer F.Cu) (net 4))
 (segment (start 175.84 92.596) (end 175.908 92.664) (width 0.25) (layer F.Cu) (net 4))
 (segment (start 175.84 90.68) (end 175.84 92.596) (width 0.25) (layer F.Cu) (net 4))
 (segment (start 180.45641 87.2) (end 181.05 87.2) (width 0.25) (layer F.Cu) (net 4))
 (segment (start 176.97641 90.68) (end 180.45641 87.2) (width 0.25) (layer F.Cu) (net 4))
 (segment (start 181.427 82.176) (end 181.45 82.199) (width 0.25) (layer F.Cu) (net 1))
 (segment (start 181.427 81.207) (end 181.427 80.726) (width 0.25) (layer F.Cu) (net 1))
 (segment (start 181.427 81.207) (end 181.427 82.176) (width 0.25) (layer F.Cu) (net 1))
 (segment (start 182.19 84.514) (end 182.19 85.66) (width 0.25) (layer F.Cu) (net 2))
 (segment (start 181.45 83.774) (end 182.19 84.514) (width 0.25) (layer F.Cu) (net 2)))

